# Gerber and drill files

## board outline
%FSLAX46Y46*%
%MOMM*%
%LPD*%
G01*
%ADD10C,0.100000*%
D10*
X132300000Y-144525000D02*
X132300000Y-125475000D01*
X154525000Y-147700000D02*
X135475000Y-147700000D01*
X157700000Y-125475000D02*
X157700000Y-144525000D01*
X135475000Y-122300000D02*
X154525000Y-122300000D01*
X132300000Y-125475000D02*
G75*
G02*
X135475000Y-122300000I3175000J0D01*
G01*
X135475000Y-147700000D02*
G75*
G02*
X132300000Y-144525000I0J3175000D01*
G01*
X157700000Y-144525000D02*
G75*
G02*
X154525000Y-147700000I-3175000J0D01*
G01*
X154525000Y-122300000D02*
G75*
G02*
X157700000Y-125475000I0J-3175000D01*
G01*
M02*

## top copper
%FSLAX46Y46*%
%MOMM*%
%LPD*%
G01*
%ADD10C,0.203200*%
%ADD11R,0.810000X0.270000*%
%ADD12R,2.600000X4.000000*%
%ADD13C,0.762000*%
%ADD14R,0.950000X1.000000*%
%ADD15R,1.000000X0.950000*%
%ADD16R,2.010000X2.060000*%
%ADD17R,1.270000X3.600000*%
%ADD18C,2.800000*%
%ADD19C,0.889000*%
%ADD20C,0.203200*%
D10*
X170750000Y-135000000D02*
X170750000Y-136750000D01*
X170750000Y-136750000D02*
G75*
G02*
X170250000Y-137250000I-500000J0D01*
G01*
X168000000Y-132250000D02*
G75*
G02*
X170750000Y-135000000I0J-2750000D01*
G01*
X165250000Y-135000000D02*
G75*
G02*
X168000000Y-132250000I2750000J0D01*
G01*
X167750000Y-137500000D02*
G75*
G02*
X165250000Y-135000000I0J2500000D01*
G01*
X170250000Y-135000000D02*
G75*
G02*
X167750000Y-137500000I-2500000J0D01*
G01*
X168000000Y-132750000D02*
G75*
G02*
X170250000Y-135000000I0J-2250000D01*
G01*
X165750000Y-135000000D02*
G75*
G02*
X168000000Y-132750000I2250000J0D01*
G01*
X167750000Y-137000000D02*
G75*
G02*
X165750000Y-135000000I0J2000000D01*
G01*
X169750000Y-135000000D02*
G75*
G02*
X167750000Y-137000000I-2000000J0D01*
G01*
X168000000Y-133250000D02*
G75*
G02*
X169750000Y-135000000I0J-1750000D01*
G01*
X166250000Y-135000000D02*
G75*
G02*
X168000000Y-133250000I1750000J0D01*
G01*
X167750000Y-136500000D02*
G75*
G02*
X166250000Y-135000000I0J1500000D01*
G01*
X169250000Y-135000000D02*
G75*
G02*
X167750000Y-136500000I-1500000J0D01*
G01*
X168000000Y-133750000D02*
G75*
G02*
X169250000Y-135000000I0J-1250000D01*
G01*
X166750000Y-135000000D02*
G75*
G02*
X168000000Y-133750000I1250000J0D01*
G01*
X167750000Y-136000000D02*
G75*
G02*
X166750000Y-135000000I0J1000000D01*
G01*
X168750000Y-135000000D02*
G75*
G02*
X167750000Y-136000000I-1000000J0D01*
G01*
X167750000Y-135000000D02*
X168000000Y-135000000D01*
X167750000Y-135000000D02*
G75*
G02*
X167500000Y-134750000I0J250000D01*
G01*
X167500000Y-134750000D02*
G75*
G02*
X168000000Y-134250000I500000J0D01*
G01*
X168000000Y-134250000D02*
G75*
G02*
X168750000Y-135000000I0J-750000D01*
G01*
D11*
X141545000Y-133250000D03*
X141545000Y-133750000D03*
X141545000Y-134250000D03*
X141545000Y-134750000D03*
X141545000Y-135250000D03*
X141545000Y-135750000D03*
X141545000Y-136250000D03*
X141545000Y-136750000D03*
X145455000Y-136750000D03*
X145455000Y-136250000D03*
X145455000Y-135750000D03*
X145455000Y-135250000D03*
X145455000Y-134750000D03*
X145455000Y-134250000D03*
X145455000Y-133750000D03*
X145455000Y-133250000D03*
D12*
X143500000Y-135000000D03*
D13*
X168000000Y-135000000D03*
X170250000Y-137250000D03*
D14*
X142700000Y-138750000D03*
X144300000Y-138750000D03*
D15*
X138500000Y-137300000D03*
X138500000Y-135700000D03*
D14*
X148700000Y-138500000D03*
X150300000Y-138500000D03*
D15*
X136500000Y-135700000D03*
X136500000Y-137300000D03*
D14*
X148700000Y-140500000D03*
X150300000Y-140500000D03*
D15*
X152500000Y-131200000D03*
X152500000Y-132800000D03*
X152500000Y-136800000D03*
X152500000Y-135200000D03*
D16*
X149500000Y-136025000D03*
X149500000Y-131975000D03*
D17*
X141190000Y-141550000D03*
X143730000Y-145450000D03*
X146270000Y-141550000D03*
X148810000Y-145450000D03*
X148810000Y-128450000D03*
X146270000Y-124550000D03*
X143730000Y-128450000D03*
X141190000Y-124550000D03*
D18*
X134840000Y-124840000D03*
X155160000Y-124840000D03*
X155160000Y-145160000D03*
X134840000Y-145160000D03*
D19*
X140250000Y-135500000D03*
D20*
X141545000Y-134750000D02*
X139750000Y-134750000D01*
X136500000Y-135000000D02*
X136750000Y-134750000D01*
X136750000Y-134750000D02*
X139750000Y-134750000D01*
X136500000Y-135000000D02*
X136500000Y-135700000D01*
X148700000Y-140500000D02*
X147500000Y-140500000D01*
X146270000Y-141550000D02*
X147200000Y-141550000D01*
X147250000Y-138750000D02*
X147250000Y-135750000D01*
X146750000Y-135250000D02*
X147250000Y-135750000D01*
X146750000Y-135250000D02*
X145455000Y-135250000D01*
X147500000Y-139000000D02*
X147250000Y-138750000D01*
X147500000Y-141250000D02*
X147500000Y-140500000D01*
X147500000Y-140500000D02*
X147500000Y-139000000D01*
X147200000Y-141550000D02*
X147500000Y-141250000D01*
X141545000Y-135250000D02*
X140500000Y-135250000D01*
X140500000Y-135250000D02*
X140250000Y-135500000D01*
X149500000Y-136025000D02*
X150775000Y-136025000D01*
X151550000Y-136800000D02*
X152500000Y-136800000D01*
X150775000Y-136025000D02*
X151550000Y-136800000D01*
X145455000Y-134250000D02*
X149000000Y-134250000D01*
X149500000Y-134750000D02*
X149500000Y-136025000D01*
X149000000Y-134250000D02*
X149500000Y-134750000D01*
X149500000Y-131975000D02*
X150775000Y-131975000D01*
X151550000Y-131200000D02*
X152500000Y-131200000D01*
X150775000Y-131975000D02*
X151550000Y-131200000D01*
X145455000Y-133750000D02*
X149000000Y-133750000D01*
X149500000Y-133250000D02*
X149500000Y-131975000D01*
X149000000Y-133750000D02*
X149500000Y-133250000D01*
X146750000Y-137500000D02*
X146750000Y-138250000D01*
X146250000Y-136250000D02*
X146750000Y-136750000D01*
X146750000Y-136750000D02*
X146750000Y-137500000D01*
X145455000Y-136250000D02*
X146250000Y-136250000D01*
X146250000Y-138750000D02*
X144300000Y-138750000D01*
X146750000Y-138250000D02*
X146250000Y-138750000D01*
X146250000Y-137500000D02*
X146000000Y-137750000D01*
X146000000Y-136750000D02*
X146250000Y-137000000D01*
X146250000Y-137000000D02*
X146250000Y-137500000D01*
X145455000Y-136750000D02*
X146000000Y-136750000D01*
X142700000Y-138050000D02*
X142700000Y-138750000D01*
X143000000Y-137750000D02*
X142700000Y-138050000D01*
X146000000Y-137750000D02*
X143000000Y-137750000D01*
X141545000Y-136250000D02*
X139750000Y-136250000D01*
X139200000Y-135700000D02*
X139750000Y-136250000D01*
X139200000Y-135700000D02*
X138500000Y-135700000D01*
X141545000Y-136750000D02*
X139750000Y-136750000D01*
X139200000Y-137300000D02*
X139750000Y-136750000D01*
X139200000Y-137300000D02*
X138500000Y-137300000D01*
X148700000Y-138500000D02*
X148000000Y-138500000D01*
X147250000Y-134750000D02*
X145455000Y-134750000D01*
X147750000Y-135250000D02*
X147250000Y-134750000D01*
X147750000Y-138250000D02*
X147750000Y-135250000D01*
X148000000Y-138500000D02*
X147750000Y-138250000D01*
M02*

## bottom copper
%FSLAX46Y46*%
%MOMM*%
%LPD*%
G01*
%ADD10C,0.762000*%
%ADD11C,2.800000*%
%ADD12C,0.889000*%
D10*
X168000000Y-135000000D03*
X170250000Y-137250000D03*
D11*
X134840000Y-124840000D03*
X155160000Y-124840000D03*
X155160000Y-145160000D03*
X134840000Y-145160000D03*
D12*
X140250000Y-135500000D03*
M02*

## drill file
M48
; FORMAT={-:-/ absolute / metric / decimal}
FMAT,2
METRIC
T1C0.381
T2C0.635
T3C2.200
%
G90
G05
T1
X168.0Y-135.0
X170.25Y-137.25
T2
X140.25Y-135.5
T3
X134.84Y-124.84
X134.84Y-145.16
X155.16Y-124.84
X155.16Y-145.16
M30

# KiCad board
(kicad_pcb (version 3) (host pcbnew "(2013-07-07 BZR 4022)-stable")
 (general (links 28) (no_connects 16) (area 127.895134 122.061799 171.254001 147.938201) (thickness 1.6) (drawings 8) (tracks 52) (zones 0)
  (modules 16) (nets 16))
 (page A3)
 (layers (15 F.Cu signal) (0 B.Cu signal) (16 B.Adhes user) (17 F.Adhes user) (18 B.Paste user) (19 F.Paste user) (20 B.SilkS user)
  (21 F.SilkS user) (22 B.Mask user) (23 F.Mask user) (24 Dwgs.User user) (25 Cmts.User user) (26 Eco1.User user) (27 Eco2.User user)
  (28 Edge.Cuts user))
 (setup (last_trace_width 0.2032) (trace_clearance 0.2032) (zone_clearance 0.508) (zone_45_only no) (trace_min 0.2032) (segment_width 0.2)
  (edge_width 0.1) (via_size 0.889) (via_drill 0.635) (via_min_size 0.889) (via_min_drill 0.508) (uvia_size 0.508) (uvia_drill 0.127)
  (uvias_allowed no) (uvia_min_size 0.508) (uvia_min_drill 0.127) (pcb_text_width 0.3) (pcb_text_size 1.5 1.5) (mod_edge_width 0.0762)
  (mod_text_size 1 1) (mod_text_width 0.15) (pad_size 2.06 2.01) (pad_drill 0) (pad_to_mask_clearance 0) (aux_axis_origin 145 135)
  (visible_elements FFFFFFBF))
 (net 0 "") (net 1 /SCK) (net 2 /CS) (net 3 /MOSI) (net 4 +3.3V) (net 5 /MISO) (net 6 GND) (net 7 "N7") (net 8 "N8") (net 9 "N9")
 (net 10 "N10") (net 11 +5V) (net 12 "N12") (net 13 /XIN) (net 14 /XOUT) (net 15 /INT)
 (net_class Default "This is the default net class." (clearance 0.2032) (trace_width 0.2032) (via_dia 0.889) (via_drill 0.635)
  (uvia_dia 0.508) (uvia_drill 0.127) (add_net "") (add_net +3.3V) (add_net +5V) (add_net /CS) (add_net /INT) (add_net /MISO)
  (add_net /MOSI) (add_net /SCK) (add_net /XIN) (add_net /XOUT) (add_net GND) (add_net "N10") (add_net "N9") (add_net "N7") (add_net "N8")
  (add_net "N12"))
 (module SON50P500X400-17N (layer F.Cu) (at 143.5 135 270)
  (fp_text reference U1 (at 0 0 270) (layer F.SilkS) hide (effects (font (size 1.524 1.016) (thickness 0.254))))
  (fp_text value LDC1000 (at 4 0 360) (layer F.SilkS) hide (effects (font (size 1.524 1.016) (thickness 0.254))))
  (pad 1 smd rect (at -1.75 1.955 270) (size 0.27 0.81) (layers F.Cu F.Paste F.Mask) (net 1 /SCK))
  (pad 2 smd rect (at -1.25 1.955 270) (size 0.27 0.81) (layers F.Cu F.Paste F.Mask) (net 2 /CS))
  (pad 3 smd rect (at -0.75 1.955 270) (size 0.27 0.81) (layers F.Cu F.Paste F.Mask) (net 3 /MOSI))
  (pad 4 smd rect (at -0.25 1.955 270) (size 0.27 0.81) (layers F.Cu F.Paste F.Mask) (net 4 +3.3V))
  (pad 5 smd rect (at 0.25 1.955 270) (size 0.27 0.81) (layers F.Cu F.Paste F.Mask) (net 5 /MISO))
  (pad 6 smd rect (at 0.75 1.955 270) (size 0.27 0.81) (layers F.Cu F.Paste F.Mask) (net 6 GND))
  (pad 7 smd rect (at 1.25 1.955 270) (size 0.27 0.81) (layers F.Cu F.Paste F.Mask) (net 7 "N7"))
  (pad 8 smd rect (at 1.75 1.955 270) (size 0.27 0.81) (layers F.Cu F.Paste F.Mask) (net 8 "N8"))
  (pad 9 smd rect (at 1.75 -1.955 270) (size 0.27 0.81) (layers F.Cu F.Paste F.Mask) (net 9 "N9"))
  (pad 10 smd rect (at 1.25 -1.955 270) (size 0.27 0.81) (layers F.Cu F.Paste F.Mask) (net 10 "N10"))
  (pad 11 smd rect (at 0.75 -1.955 270) (size 0.27 0.81) (layers F.Cu F.Paste F.Mask) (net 6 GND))
  (pad 12 smd rect (at 0.25 -1.955 270) (size 0.27 0.81) (layers F.Cu F.Paste F.Mask) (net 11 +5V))
  (pad 13 smd rect (at -0.25 -1.955 270) (size 0.27 0.81) (layers F.Cu F.Paste F.Mask) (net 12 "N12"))
  (pad 14 smd rect (at -0.75 -1.955 270) (size 0.27 0.81) (layers F.Cu F.Paste F.Mask) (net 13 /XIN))
  (pad 15 smd rect (at -1.25 -1.955 270) (size 0.27 0.81) (layers F.Cu F.Paste F.Mask) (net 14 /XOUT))
  (pad 16 smd rect (at -1.75 -1.955 270) (size 0.27 0.81) (layers F.Cu F.Paste F.Mask) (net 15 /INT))
  (pad 17 smd rect (at 0 0 270) (size 4 2.6) (layers F.Cu F.Paste F.Mask) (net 6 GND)))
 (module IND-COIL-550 (layer F.Cu) (at 168 135) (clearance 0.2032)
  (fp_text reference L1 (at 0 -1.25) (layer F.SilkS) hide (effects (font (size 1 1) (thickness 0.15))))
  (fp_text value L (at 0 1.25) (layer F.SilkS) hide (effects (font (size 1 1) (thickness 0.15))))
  (fp_line (start 2.75 0) (end 2.75 1.75) (layer F.Cu) (width 0.2032))
  (fp_arc (start 2.25 1.75) (end 2.75 1.75) (angle 90) (layer F.Cu) (width 0.2032))
  (fp_arc (start 0 0) (end 0 -2.75) (angle 90) (layer F.Cu) (width 0.2032))
  (fp_arc (start 0 0) (end -2.75 0) (angle 90) (layer F.Cu) (width 0.2032))
  (fp_arc (start -0.25 0) (end -0.25 2.5) (angle 90) (layer F.Cu) (width 0.2032))
  (fp_arc (start -0.25 0) (end 2.25 0) (angle 90) (layer F.Cu) (width 0.2032))
  (fp_arc (start 0 0) (end 0 -2.25) (angle 90) (layer F.Cu) (width 0.2032))
  (fp_arc (start 0 0) (end -2.25 0) (angle 90) (layer F.Cu) (width 0.2032))
  (fp_arc (start -0.25 0) (end -0.25 2) (angle 90) (layer F.Cu) (width 0.2032))
  (fp_arc (start -0.25 0) (end 1.75 0) (angle 90) (layer F.Cu) (width 0.2032))
  (fp_arc (start 0 0) (end 0 -1.75) (angle 90) (layer F.Cu) (width 0.2032))
  (fp_arc (start 0 0) (end -1.75 0) (angle 90) (layer F.Cu) (width 0.2032))
  (fp_arc (start -0.25 0) (end -0.25 1.5) (angle 90) (layer F.Cu) (width 0.2032))
  (fp_arc (start -0.25 0) (end 1.25 0) (angle 90) (layer F.Cu) (width 0.2032))
  (fp_arc (start 0 0) (end 0 -1.25) (angle 90) (layer F.Cu) (width 0.2032))
  (fp_arc (start 0 0) (end -1.25 0) (angle 90) (layer F.Cu) (width 0.2032))
  (fp_arc (start -0.25 0) (end -0.25 1) (angle 90) (layer F.Cu) (width 0.2032))
  (fp_arc (start -0.25 0) (end 0.75 0) (angle 90) (layer F.Cu) (width 0.2032))
  (fp_line (start -0.25 0) (end 0 0) (layer F.Cu) (width 0.2032))
  (fp_arc (start -0.25 -0.25) (end -0.25 0) (angle 90) (layer F.Cu) (width 0.2032))
  (fp_arc (start 0 -0.25) (end -0.5 -0.25) (angle 90) (layer F.Cu) (width 0.2032))
  (fp_arc (start 0 0) (end 0 -0.75) (angle 90) (layer F.Cu) (width 0.2032))
  (pad 1 thru_hole circle (at 0 0) (size 0.762 0.762) (drill 0.381) (layers *.Cu *.Mask F.SilkS) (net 10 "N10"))
  (pad 2 thru_hole circle (at 2.25 2.25) (size 0.762 0.762) (drill 0.381) (layers *.Cu *.Mask F.SilkS) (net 9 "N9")))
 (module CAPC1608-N (layer F.Cu) (at 143.5 138.75)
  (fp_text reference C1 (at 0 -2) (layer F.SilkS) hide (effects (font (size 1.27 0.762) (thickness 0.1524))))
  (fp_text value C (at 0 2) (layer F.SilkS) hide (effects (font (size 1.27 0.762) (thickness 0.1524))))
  (pad 1 smd rect (at -0.8 0) (size 0.95 1) (layers F.Cu F.Paste F.Mask) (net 9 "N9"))
  (pad 2 smd rect (at 0.8 0) (size 0.95 1) (layers F.Cu F.Paste F.Mask) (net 10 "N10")))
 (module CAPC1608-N (layer F.Cu) (at 138.5 136.5 90)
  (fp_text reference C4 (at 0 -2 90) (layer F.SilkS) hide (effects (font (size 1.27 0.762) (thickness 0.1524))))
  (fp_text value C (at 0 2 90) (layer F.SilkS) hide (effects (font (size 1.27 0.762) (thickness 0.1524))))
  (pad 1 smd rect (at -0.8 0 90) (size 0.95 1) (layers F.Cu F.Paste F.Mask) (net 8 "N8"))
  (pad 2 smd rect (at 0.8 0 90) (size 0.95 1) (layers F.Cu F.Paste F.Mask) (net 7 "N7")))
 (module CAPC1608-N (layer F.Cu) (at 149.5 138.5)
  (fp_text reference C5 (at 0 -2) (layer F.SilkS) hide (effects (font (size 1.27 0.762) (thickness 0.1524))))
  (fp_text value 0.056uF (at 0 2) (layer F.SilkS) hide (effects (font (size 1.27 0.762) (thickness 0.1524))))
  (pad 1 smd rect (at -0.8 0) (size 0.95 1) (layers F.Cu F.Paste F.Mask) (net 12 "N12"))
  (pad 2 smd rect (at 0.8 0) (size 0.95 1) (layers F.Cu F.Paste F.Mask) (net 6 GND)))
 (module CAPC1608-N (layer F.Cu) (at 136.5 136.5 270)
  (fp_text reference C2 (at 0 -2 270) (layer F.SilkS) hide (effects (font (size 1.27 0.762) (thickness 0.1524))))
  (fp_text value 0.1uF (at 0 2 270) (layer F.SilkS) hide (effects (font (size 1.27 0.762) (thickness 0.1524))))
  (pad 1 smd rect (at -0.8 0 270) (size 0.95 1) (layers F.Cu F.Paste F.Mask) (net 4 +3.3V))
  (pad 2 smd rect (at 0.8 0 270) (size 0.95 1) (layers F.Cu F.Paste F.Mask) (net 6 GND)))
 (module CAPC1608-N (layer F.Cu) (at 149.5 140.5)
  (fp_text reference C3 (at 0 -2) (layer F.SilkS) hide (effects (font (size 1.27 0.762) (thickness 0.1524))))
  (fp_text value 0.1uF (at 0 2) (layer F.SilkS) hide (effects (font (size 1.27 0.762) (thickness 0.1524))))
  (pad 1 smd rect (at -0.8 0) (size 0.95 1) (layers F.Cu F.Paste F.Mask) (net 11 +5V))
  (pad 2 smd rect (at 0.8 0) (size 0.95 1) (layers F.Cu F.Paste F.Mask) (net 6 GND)))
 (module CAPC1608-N (layer F.Cu) (at 152.5 132 270)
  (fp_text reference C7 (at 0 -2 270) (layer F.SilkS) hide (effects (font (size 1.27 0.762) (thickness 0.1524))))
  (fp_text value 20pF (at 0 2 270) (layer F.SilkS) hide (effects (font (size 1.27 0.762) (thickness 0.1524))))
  (pad 1 smd rect (at -0.8 0 270) (size 0.95 1) (layers F.Cu F.Paste F.Mask) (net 14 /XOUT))
  (pad 2 smd rect (at 0.8 0 270) (size 0.95 1) (layers F.Cu F.Paste F.Mask) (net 6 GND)))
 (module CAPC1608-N (layer F.Cu) (at 152.5 136 90)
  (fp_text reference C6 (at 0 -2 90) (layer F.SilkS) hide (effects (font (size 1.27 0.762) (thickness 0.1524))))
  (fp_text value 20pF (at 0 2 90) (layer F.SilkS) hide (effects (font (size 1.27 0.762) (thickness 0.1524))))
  (pad 1 smd rect (at -0.8 0 90) (size 0.95 1) (layers F.Cu F.Paste F.Mask) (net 13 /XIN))
  (pad 2 smd rect (at 0.8 0 90) (size 0.95 1) (layers F.Cu F.Paste F.Mask) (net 6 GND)))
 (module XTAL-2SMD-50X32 (layer F.Cu) (at 149.5 134 90)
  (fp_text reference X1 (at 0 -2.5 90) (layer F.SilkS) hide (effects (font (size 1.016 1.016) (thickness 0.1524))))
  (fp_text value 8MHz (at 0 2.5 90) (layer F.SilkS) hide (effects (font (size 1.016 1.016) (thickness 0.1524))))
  (pad 1 smd rect (at -2.025 0 90) (size 2.06 2.01) (layers F.Cu F.Paste F.Mask) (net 13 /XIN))
  (pad 2 smd rect (at 2.025 0 90) (size 2.06 2.01) (layers F.Cu F.Paste F.Mask) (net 14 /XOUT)))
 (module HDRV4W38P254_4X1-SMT (layer F.Cu) (at 145 143.5)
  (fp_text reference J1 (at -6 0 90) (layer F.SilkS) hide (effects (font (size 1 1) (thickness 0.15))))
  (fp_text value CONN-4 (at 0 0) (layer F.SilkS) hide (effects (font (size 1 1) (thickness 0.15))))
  (pad 1 smd rect (at -3.81 -1.95) (size 1.27 3.6) (layers F.Cu F.Paste F.Mask) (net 4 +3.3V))
  (pad 2 smd rect (at -1.27 1.95) (size 1.27 3.6) (layers F.Cu F.Paste F.Mask) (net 6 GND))
  (pad 3 smd rect (at 1.27 -1.95) (size 1.27 3.6) (layers F.Cu F.Paste F.Mask) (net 11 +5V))
  (pad 4 smd rect (at 3.81 1.95) (size 1.27 3.6) (layers F.Cu F.Paste F.Mask) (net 15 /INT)))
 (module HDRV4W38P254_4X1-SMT (layer F.Cu) (at 145 126.5 180)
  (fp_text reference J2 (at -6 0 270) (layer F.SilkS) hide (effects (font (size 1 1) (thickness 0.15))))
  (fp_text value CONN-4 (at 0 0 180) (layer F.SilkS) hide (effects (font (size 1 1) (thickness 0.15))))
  (pad 1 smd rect (at -3.81 -1.95 180) (size 1.27 3.6) (layers F.Cu F.Paste F.Mask) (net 1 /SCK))
  (pad 2 smd rect (at -1.27 1.95 180) (size 1.27 3.6) (layers F.Cu F.Paste F.Mask) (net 2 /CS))
  (pad 3 smd rect (at 1.27 -1.95 180) (size 1.27 3.6) (layers F.Cu F.Paste F.Mask) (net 3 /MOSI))
  (pad 4 smd rect (at 3.81 1.95 180) (size 1.27 3.6) (layers F.Cu F.Paste F.Mask) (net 5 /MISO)))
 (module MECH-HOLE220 (layer F.Cu) (at 134.84 124.84)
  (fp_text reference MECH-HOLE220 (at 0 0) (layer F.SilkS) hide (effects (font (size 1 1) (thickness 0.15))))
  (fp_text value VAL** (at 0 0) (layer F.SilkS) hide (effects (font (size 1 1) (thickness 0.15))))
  (pad "" thru_hole circle (at 0 0) (size 2.8 2.8) (drill 2.2) (layers *.Cu *.Mask F.SilkS)))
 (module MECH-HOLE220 (layer F.Cu) (at 155.16 124.84)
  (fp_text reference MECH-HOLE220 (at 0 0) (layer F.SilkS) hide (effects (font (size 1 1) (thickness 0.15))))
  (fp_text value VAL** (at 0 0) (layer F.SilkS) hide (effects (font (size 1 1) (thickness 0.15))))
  (pad "" thru_hole circle (at 0 0) (size 2.8 2.8) (drill 2.2) (layers *.Cu *.Mask F.SilkS)))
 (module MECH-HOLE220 (layer F.Cu) (at 155.16 145.16)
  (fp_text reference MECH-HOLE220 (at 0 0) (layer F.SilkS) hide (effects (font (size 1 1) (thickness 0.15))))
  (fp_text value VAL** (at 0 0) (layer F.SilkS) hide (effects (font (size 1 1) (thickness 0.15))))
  (pad "" thru_hole circle (at 0 0) (size 2.8 2.8) (drill 2.2) (layers *.Cu *.Mask F.SilkS)))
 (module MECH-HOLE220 (layer F.Cu) (at 134.84 145.16)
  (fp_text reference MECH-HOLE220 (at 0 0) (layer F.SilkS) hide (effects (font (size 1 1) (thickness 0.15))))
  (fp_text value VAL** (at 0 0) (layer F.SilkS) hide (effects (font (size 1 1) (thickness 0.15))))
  (pad "" thru_hole circle (at 0 0) (size 2.8 2.8) (drill 2.2) (layers *.Cu *.Mask F.SilkS)))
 (gr_line (start 132.3 144.525) (end 132.3 125.475) (angle 90) (layer Edge.Cuts) (width 0.1))
 (gr_line (start 154.525 147.7) (end 135.475 147.7) (angle 90) (layer Edge.Cuts) (width 0.1))
 (gr_line (start 157.7 125.475) (end 157.7 144.525) (angle 90) (layer Edge.Cuts) (width 0.1))
 (gr_line (start 135.475 122.3) (end 154.525 122.3) (angle 90) (layer Edge.Cuts) (width 0.1))
 (gr_arc (start 135.475 125.475) (end 132.3 125.475) (angle 90) (layer Edge.Cuts) (width 0.1))
 (gr_arc (start 135.475 144.525) (end 135.475 147.7) (angle 90) (layer Edge.Cuts) (width 0.1))
 (gr_arc (start 154.525 144.525) (end 157.7 144.525) (angle 90) (layer Edge.Cuts) (width 0.1))
 (gr_arc (start 154.525 125.475) (end 154.525 122.3) (angle 90) (layer Edge.Cuts) (width 0.1))
 (segment (start 141.545 134.75) (end 139.75 134.75) (width 0.2032) (layer F.Cu) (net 4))
 (segment (start 136.5 135) (end 136.75 134.75) (width 0.2032) (layer F.Cu) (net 4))
 (segment (start 136.75 134.75) (end 139.75 134.75) (width 0.2032) (layer F.Cu) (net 4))
 (segment (start 136.5 135) (end 136.5 135.7) (width 0.2032) (layer F.Cu) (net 4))
 (segment (start 148.7 140.5) (end 147.5 140.5) (width 0.2032) (layer F.Cu) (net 11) (status 400000))
 (segment (start 146.27 141.55) (end 147.2 141.55) (width 0.2032) (layer F.Cu) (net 11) (status 400000))
 (segment (start 147.25 138.75) (end 147.25 135.75) (width 0.2032) (layer F.Cu) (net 11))
 (segment (start 146.75 135.25) (end 147.25 135.75) (width 0.2032) (layer F.Cu) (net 11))
 (segment (start 146.75 135.25) (end 145.455 135.25) (width 0.2032) (layer F.Cu) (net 11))
 (segment (start 147.5 139) (end 147.25 138.75) (width 0.2032) (layer F.Cu) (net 11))
 (segment (start 147.5 141.25) (end 147.5 140.5) (width 0.2032) (layer F.Cu) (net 11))
 (segment (start 147.5 140.5) (end 147.5 139) (width 0.2032) (layer F.Cu) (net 11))
 (segment (start 147.2 141.55) (end 147.5 141.25) (width 0.2032) (layer F.Cu) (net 11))
 (segment (start 141.545 135.25) (end 140.5 135.25) (width 0.2032) (layer F.Cu) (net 5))
 (via (at 140.25 135.5) (size 0.889) (layers F.Cu B.Cu) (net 5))
 (segment (start 140.5 135.25) (end 140.25 135.5) (width 0.2032) (layer F.Cu) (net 5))
 (segment (start 149.5 136.025) (end 150.775 136.025) (width 0.2032) (layer F.Cu) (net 13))
 (segment (start 151.55 136.8) (end 152.5 136.8) (width 0.2032) (layer F.Cu) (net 13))
 (segment (start 150.775 136.025) (end 151.55 136.8) (width 0.2032) (layer F.Cu) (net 13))
 (segment (start 145.455 134.25) (end 149 134.25) (width 0.2032) (layer F.Cu) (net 13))
 (segment (start 149.5 134.75) (end 149.5 136.025) (width 0.2032) (layer F.Cu) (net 13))
 (segment (start 149 134.25) (end 149.5 134.75) (width 0.2032) (layer F.Cu) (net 13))
 (segment (start 149.5 131.975) (end 150.775 131.975) (width 0.2032) (layer F.Cu) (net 14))
 (segment (start 151.55 131.2) (end 152.5 131.2) (width 0.2032) (layer F.Cu) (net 14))
 (segment (start 150.775 131.975) (end 151.55 131.2) (width 0.2032) (layer F.Cu) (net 14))
 (segment (start 145.455 133.75) (end 149 133.75) (width 0.2032) (layer F.Cu) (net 14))
 (segment (start 149.5 133.25) (end 149.5 131.975) (width 0.2032) (layer F.Cu) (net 14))
 (segment (start 149 133.75) (end 149.5 133.25) (width 0.2032) (layer F.Cu) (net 14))
 (segment (start 146.75 137.5) (end 146.75 138.25) (width 0.2032) (layer F.Cu) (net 10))
 (segment (start 146.25 136.25) (end 146.75 136.75) (width 0.2032) (layer F.Cu) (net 10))
 (segment (start 146.75 136.75) (end 146.75 137.5) (width 0.2032) (layer F.Cu) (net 10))
 (segment (start 145.455 136.25) (end 146.25 136.25) (width 0.2032) (layer F.Cu) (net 10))
 (segment (start 146.25 138.75) (end 144.3 138.75) (width 0.2032) (layer F.Cu) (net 10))
 (segment (start 146.75 138.25) (end 146.25 138.75) (width 0.2032) (layer F.Cu) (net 10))
 (segment (start 146.25 137.5) (end 146 137.75) (width 0.2032) (layer F.Cu) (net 9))
 (segment (start 146 136.75) (end 146.25 137) (width 0.2032) (layer F.Cu) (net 9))
 (segment (start 146.25 137) (end 146.25 137.5) (width 0.2032) (layer F.Cu) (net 9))
 (segment (start 145.455 136.75) (end 146 136.75) (width 0.2032) (layer F.Cu) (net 9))
 (segment (start 142.7 138.05) (end 142.7 138.75) (width 0.2032) (layer F.Cu) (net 9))
 (segment (start 143 137.75) (end 142.7 138.05) (width 0.2032) (layer F.Cu) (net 9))
 (segment (start 146 137.75) (end 143 137.75) (width 0.2032) (layer F.Cu) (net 9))
 (segment (start 141.545 136.25) (end 139.75 136.25) (width 0.2032) (layer F.Cu) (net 7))
 (segment (start 139.2 135.7) (end 139.75 136.25) (width 0.2032) (layer F.Cu) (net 7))
 (segment (start 139.2 135.7) (end 138.5 135.7) (width 0.2032) (layer F.Cu) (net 7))
 (segment (start 141.545 136.75) (end 139.75 136.75) (width 0.2032) (layer F.Cu) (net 8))
 (segment (start 139.2 137.3) (end 139.75 136.75) (width 0.2032) (layer F.Cu) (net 8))
 (segment (start 139.2 137.3) (end 138.5 137.3) (width 0.2032) (layer F.Cu) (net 8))
 (segment (start 148.7 138.5) (end 148 138.5) (width 0.2032) (layer F.Cu) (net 12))
 (segment (start 147.25 134.75) (end 145.455 134.75) (width 0.2032) (layer F.Cu) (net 12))
 (segment (start 147.75 135.25) (end 147.25 134.75) (width 0.2032) (layer F.Cu) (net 12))
 (segment (start 147.75 138.25) (end 147.75 135.25) (width 0.2032) (layer F.Cu) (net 12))
 (segment (start 148 138.5) (end 147.75 138.25) (width 0.2032) (layer F.Cu) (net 12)))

